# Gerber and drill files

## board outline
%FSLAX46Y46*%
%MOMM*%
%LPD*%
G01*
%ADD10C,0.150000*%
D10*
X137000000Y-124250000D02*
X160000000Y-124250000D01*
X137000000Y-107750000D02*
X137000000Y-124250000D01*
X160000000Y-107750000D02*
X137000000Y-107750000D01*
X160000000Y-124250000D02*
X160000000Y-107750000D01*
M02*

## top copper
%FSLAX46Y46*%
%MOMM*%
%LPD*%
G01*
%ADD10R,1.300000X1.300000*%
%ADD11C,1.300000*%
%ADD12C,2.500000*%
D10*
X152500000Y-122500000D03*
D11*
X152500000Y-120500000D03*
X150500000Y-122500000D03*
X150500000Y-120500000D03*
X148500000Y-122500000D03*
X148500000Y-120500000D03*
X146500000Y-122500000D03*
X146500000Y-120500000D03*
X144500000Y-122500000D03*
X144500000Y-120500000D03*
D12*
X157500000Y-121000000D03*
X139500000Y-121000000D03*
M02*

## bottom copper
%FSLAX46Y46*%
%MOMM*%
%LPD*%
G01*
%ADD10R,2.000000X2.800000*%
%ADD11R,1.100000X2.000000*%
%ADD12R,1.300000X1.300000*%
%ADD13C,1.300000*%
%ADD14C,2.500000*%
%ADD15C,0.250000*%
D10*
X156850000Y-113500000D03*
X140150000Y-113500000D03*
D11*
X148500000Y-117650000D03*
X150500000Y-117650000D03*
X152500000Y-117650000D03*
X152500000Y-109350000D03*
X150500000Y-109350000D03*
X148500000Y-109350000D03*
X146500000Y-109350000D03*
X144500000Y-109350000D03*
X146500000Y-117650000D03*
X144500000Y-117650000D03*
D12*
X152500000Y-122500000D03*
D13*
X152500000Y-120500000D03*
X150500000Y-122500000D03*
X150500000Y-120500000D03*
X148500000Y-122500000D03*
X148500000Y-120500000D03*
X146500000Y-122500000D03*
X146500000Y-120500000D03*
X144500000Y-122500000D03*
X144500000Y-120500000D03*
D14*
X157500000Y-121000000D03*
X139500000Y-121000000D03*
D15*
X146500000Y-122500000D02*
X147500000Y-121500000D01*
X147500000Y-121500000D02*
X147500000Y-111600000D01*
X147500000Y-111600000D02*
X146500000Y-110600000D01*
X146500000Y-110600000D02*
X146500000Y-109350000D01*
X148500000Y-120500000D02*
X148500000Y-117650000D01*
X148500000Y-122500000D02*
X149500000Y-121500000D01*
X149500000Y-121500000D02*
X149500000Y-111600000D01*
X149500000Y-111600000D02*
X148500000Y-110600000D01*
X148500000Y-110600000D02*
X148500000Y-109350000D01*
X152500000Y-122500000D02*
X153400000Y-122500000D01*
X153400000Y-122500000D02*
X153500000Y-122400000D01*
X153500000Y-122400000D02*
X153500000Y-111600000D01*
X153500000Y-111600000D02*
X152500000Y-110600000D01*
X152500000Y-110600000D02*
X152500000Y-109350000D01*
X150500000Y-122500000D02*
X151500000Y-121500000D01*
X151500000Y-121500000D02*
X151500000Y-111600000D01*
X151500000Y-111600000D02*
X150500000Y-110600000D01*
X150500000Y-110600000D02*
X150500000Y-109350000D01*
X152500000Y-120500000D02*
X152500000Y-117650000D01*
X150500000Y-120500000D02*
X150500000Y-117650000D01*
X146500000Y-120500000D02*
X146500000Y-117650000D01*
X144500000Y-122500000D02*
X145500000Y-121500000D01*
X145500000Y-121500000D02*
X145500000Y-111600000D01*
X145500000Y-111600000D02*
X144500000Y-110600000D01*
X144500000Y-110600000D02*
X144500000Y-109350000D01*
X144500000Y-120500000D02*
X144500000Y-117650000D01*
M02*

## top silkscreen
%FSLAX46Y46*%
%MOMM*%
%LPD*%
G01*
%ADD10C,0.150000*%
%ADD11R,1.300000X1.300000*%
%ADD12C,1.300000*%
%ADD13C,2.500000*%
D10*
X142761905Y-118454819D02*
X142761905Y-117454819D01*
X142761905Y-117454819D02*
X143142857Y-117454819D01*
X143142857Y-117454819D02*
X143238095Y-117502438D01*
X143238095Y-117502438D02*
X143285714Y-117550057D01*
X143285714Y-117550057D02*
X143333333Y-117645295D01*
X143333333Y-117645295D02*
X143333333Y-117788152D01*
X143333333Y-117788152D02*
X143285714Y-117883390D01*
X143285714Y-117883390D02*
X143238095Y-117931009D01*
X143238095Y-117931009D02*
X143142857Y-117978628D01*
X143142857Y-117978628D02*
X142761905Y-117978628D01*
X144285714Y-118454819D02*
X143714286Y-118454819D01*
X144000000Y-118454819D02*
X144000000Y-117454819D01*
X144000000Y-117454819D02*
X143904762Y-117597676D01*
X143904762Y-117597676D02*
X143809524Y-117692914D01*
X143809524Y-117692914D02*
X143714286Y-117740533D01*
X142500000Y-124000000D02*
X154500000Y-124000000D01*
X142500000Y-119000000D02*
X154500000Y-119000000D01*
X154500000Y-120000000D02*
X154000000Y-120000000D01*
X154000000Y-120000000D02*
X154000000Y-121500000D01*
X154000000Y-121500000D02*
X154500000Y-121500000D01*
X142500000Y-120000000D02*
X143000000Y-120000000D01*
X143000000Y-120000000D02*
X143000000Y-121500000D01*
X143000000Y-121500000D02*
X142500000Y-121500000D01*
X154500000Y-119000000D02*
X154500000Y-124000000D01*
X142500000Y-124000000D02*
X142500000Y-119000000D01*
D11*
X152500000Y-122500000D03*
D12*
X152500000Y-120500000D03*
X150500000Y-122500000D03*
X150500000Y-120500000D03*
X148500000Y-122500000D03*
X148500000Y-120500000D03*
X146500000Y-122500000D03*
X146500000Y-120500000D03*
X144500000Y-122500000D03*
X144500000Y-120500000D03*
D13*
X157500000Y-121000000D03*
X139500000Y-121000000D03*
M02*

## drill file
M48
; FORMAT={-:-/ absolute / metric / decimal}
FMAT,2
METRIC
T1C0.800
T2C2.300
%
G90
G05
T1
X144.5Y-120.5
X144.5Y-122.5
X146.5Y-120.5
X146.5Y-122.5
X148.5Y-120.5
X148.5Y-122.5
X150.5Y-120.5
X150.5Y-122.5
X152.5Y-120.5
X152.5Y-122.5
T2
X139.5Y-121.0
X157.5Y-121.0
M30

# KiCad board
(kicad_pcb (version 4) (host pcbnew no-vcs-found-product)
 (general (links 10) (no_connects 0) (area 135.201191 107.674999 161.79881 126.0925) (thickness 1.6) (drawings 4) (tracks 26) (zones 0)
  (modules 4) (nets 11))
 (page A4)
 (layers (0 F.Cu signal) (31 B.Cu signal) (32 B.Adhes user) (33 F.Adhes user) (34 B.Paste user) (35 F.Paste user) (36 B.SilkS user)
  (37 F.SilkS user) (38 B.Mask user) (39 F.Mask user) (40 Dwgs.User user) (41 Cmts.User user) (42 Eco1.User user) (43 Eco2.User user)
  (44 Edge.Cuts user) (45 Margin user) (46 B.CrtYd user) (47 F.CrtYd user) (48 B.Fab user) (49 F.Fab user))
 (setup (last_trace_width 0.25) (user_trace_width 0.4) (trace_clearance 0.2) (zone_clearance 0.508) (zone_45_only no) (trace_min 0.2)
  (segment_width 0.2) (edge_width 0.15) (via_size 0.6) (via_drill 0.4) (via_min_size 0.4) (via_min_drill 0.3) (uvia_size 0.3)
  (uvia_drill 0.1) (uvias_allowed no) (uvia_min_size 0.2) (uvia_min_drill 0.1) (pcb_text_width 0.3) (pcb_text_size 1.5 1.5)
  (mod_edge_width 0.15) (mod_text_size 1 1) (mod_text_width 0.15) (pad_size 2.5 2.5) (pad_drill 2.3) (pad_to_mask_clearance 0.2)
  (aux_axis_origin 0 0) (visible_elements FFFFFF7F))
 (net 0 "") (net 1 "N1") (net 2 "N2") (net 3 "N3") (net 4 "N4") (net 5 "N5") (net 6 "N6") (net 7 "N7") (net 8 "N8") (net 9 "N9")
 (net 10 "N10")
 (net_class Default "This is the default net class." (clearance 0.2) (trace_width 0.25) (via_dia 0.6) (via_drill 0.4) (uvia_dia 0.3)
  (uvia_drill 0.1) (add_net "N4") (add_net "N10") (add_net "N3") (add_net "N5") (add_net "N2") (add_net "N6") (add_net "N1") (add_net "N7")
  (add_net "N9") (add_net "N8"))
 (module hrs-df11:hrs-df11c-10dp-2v (layer B.Cu) (at 148.5 113.5)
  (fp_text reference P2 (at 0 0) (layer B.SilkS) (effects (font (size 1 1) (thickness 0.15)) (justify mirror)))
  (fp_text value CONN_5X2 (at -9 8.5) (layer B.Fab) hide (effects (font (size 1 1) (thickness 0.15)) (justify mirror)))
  (pad "" smd rect (at 8.35 0) (size 2 2.8) (layers B.Cu B.Paste B.Mask))
  (pad "" smd rect (at -8.35 0) (size 2 2.8) (layers B.Cu B.Paste B.Mask))
  (pad 6 smd rect (at 0 4.15) (size 1.1 2) (layers B.Cu B.Paste B.Mask) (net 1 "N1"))
  (pad 4 smd rect (at 2 4.15) (size 1.1 2) (layers B.Cu B.Paste B.Mask) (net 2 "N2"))
  (pad 2 smd rect (at 4 4.15) (size 1.1 2) (layers B.Cu B.Paste B.Mask) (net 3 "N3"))
  (pad 1 smd rect (at 4 -4.15) (size 1.1 2) (layers B.Cu B.Paste B.Mask) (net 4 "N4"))
  (pad 3 smd rect (at 2 -4.15) (size 1.1 2) (layers B.Cu B.Paste B.Mask) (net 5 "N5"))
  (pad 5 smd rect (at 0 -4.15) (size 1.1 2) (layers B.Cu B.Paste B.Mask) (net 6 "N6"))
  (pad 7 smd rect (at -2 -4.15) (size 1.1 2) (layers B.Cu B.Paste B.Mask) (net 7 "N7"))
  (pad 9 smd rect (at -4 -4.15) (size 1.1 2) (layers B.Cu B.Paste B.Mask) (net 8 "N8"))
  (pad 8 smd rect (at -2 4.15) (size 1.1 2) (layers B.Cu B.Paste B.Mask) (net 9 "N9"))
  (pad 10 smd rect (at -4 4.15) (size 1.1 2) (layers B.Cu B.Paste B.Mask) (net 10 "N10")))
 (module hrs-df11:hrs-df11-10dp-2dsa (layer F.Cu) (at 148.5 121.5)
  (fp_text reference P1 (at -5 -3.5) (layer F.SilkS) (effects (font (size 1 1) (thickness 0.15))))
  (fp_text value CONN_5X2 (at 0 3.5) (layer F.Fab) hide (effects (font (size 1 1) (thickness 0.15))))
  (fp_line (start -6 2.5) (end 6 2.5) (layer F.SilkS) (width 0.15))
  (fp_line (start -6 -2.5) (end 6 -2.5) (layer F.SilkS) (width 0.15))
  (fp_line (start 6 -1.5) (end 5.5 -1.5) (layer F.SilkS) (width 0.15))
  (fp_line (start 5.5 -1.5) (end 5.5 0) (layer F.SilkS) (width 0.15))
  (fp_line (start 5.5 0) (end 6 0) (layer F.SilkS) (width 0.15))
  (fp_line (start -6 -1.5) (end -5.5 -1.5) (layer F.SilkS) (width 0.15))
  (fp_line (start -5.5 -1.5) (end -5.5 0) (layer F.SilkS) (width 0.15))
  (fp_line (start -5.5 0) (end -6 0) (layer F.SilkS) (width 0.15))
  (fp_line (start 6 -2.5) (end 6 2.5) (layer F.SilkS) (width 0.15))
  (fp_line (start -6 2.5) (end -6 -2.5) (layer F.SilkS) (width 0.15))
  (pad 1 thru_hole rect (at 4 1) (size 1.3 1.3) (drill 0.8) (layers *.Cu *.Mask F.SilkS) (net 4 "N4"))
  (pad 2 thru_hole circle (at 4 -1) (size 1.3 1.3) (drill 0.8) (layers *.Cu *.Mask F.SilkS) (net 3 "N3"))
  (pad 3 thru_hole circle (at 2 1) (size 1.3 1.3) (drill 0.8) (layers *.Cu *.Mask F.SilkS) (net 5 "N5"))
  (pad 4 thru_hole circle (at 2 -1) (size 1.3 1.3) (drill 0.8) (layers *.Cu *.Mask F.SilkS) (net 2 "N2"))
  (pad 5 thru_hole circle (at 0 1) (size 1.3 1.3) (drill 0.8) (layers *.Cu *.Mask F.SilkS) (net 6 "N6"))
  (pad 6 thru_hole circle (at 0 -1) (size 1.3 1.3) (drill 0.8) (layers *.Cu *.Mask F.SilkS) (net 1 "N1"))
  (pad 7 thru_hole circle (at -2 1) (size 1.3 1.3) (drill 0.8) (layers *.Cu *.Mask F.SilkS) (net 7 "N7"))
  (pad 8 thru_hole circle (at -2 -1) (size 1.3 1.3) (drill 0.8) (layers *.Cu *.Mask F.SilkS) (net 9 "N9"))
  (pad 9 thru_hole circle (at -4 1) (size 1.3 1.3) (drill 0.8) (layers *.Cu *.Mask F.SilkS) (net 8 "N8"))
  (pad 10 thru_hole circle (at -4 -1) (size 1.3 1.3) (drill 0.8) (layers *.Cu *.Mask F.SilkS) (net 10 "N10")))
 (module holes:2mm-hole (layer F.Cu) (at 157.5 121)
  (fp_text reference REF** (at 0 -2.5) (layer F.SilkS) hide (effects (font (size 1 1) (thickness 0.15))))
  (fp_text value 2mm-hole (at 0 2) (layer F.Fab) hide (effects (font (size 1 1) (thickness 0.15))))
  (pad 1 thru_hole circle (at 0 0) (size 2.5 2.5) (drill 2.3) (layers *.Cu *.Mask F.SilkS)))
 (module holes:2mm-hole (layer F.Cu) (at 139.5 121)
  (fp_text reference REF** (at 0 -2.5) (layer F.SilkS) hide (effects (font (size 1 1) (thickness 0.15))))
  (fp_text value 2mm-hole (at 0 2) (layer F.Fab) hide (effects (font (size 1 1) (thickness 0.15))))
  (pad 1 thru_hole circle (at 0 0) (size 2.5 2.5) (drill 2.3) (layers *.Cu *.Mask F.SilkS)))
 (gr_line (start 137 124.25) (end 160 124.25) (layer Edge.Cuts) (width 0.15))
 (gr_line (start 137 107.75) (end 137 124.25) (layer Edge.Cuts) (width 0.15))
 (gr_line (start 160 107.75) (end 137 107.75) (layer Edge.Cuts) (width 0.15))
 (gr_line (start 160 124.25) (end 160 107.75) (layer Edge.Cuts) (width 0.15))
 (segment (start 146.5 122.5) (end 147.5 121.5) (width 0.25) (layer B.Cu) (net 7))
 (segment (start 147.5 121.5) (end 147.5 111.6) (width 0.25) (layer B.Cu) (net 7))
 (segment (start 147.5 111.6) (end 146.5 110.6) (width 0.25) (layer B.Cu) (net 7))
 (segment (start 146.5 110.6) (end 146.5 109.35) (width 0.25) (layer B.Cu) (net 7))
 (segment (start 148.5 120.5) (end 148.5 117.65) (width 0.25) (layer B.Cu) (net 1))
 (segment (start 148.5 122.5) (end 149.5 121.5) (width 0.25) (layer B.Cu) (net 6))
 (segment (start 149.5 121.5) (end 149.5 111.6) (width 0.25) (layer B.Cu) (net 6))
 (segment (start 149.5 111.6) (end 148.5 110.6) (width 0.25) (layer B.Cu) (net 6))
 (segment (start 148.5 110.6) (end 148.5 109.35) (width 0.25) (layer B.Cu) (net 6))
 (segment (start 152.5 122.5) (end 153.4 122.5) (width 0.25) (layer B.Cu) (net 4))
 (segment (start 153.4 122.5) (end 153.5 122.4) (width 0.25) (layer B.Cu) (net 4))
 (segment (start 153.5 122.4) (end 153.5 111.6) (width 0.25) (layer B.Cu) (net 4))
 (segment (start 153.5 111.6) (end 152.5 110.6) (width 0.25) (layer B.Cu) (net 4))
 (segment (start 152.5 110.6) (end 152.5 109.35) (width 0.25) (layer B.Cu) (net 4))
 (segment (start 150.5 122.5) (end 151.5 121.5) (width 0.25) (layer B.Cu) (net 5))
 (segment (start 151.5 121.5) (end 151.5 111.6) (width 0.25) (layer B.Cu) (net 5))
 (segment (start 151.5 111.6) (end 150.5 110.6) (width 0.25) (layer B.Cu) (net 5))
 (segment (start 150.5 110.6) (end 150.5 109.35) (width 0.25) (layer B.Cu) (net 5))
 (segment (start 152.5 120.5) (end 152.5 117.65) (width 0.25) (layer B.Cu) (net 3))
 (segment (start 150.5 120.5) (end 150.5 117.65) (width 0.25) (layer B.Cu) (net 2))
 (segment (start 146.5 120.5) (end 146.5 117.65) (width 0.25) (layer B.Cu) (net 9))
 (segment (start 144.5 122.5) (end 145.5 121.5) (width 0.25) (layer B.Cu) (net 8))
 (segment (start 145.5 121.5) (end 145.5 111.6) (width 0.25) (layer B.Cu) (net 8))
 (segment (start 145.5 111.6) (end 144.5 110.6) (width 0.25) (layer B.Cu) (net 8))
 (segment (start 144.5 110.6) (end 144.5 109.35) (width 0.25) (layer B.Cu) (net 8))
 (segment (start 144.5 120.5) (end 144.5 117.65) (width 0.25) (layer B.Cu) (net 10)))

